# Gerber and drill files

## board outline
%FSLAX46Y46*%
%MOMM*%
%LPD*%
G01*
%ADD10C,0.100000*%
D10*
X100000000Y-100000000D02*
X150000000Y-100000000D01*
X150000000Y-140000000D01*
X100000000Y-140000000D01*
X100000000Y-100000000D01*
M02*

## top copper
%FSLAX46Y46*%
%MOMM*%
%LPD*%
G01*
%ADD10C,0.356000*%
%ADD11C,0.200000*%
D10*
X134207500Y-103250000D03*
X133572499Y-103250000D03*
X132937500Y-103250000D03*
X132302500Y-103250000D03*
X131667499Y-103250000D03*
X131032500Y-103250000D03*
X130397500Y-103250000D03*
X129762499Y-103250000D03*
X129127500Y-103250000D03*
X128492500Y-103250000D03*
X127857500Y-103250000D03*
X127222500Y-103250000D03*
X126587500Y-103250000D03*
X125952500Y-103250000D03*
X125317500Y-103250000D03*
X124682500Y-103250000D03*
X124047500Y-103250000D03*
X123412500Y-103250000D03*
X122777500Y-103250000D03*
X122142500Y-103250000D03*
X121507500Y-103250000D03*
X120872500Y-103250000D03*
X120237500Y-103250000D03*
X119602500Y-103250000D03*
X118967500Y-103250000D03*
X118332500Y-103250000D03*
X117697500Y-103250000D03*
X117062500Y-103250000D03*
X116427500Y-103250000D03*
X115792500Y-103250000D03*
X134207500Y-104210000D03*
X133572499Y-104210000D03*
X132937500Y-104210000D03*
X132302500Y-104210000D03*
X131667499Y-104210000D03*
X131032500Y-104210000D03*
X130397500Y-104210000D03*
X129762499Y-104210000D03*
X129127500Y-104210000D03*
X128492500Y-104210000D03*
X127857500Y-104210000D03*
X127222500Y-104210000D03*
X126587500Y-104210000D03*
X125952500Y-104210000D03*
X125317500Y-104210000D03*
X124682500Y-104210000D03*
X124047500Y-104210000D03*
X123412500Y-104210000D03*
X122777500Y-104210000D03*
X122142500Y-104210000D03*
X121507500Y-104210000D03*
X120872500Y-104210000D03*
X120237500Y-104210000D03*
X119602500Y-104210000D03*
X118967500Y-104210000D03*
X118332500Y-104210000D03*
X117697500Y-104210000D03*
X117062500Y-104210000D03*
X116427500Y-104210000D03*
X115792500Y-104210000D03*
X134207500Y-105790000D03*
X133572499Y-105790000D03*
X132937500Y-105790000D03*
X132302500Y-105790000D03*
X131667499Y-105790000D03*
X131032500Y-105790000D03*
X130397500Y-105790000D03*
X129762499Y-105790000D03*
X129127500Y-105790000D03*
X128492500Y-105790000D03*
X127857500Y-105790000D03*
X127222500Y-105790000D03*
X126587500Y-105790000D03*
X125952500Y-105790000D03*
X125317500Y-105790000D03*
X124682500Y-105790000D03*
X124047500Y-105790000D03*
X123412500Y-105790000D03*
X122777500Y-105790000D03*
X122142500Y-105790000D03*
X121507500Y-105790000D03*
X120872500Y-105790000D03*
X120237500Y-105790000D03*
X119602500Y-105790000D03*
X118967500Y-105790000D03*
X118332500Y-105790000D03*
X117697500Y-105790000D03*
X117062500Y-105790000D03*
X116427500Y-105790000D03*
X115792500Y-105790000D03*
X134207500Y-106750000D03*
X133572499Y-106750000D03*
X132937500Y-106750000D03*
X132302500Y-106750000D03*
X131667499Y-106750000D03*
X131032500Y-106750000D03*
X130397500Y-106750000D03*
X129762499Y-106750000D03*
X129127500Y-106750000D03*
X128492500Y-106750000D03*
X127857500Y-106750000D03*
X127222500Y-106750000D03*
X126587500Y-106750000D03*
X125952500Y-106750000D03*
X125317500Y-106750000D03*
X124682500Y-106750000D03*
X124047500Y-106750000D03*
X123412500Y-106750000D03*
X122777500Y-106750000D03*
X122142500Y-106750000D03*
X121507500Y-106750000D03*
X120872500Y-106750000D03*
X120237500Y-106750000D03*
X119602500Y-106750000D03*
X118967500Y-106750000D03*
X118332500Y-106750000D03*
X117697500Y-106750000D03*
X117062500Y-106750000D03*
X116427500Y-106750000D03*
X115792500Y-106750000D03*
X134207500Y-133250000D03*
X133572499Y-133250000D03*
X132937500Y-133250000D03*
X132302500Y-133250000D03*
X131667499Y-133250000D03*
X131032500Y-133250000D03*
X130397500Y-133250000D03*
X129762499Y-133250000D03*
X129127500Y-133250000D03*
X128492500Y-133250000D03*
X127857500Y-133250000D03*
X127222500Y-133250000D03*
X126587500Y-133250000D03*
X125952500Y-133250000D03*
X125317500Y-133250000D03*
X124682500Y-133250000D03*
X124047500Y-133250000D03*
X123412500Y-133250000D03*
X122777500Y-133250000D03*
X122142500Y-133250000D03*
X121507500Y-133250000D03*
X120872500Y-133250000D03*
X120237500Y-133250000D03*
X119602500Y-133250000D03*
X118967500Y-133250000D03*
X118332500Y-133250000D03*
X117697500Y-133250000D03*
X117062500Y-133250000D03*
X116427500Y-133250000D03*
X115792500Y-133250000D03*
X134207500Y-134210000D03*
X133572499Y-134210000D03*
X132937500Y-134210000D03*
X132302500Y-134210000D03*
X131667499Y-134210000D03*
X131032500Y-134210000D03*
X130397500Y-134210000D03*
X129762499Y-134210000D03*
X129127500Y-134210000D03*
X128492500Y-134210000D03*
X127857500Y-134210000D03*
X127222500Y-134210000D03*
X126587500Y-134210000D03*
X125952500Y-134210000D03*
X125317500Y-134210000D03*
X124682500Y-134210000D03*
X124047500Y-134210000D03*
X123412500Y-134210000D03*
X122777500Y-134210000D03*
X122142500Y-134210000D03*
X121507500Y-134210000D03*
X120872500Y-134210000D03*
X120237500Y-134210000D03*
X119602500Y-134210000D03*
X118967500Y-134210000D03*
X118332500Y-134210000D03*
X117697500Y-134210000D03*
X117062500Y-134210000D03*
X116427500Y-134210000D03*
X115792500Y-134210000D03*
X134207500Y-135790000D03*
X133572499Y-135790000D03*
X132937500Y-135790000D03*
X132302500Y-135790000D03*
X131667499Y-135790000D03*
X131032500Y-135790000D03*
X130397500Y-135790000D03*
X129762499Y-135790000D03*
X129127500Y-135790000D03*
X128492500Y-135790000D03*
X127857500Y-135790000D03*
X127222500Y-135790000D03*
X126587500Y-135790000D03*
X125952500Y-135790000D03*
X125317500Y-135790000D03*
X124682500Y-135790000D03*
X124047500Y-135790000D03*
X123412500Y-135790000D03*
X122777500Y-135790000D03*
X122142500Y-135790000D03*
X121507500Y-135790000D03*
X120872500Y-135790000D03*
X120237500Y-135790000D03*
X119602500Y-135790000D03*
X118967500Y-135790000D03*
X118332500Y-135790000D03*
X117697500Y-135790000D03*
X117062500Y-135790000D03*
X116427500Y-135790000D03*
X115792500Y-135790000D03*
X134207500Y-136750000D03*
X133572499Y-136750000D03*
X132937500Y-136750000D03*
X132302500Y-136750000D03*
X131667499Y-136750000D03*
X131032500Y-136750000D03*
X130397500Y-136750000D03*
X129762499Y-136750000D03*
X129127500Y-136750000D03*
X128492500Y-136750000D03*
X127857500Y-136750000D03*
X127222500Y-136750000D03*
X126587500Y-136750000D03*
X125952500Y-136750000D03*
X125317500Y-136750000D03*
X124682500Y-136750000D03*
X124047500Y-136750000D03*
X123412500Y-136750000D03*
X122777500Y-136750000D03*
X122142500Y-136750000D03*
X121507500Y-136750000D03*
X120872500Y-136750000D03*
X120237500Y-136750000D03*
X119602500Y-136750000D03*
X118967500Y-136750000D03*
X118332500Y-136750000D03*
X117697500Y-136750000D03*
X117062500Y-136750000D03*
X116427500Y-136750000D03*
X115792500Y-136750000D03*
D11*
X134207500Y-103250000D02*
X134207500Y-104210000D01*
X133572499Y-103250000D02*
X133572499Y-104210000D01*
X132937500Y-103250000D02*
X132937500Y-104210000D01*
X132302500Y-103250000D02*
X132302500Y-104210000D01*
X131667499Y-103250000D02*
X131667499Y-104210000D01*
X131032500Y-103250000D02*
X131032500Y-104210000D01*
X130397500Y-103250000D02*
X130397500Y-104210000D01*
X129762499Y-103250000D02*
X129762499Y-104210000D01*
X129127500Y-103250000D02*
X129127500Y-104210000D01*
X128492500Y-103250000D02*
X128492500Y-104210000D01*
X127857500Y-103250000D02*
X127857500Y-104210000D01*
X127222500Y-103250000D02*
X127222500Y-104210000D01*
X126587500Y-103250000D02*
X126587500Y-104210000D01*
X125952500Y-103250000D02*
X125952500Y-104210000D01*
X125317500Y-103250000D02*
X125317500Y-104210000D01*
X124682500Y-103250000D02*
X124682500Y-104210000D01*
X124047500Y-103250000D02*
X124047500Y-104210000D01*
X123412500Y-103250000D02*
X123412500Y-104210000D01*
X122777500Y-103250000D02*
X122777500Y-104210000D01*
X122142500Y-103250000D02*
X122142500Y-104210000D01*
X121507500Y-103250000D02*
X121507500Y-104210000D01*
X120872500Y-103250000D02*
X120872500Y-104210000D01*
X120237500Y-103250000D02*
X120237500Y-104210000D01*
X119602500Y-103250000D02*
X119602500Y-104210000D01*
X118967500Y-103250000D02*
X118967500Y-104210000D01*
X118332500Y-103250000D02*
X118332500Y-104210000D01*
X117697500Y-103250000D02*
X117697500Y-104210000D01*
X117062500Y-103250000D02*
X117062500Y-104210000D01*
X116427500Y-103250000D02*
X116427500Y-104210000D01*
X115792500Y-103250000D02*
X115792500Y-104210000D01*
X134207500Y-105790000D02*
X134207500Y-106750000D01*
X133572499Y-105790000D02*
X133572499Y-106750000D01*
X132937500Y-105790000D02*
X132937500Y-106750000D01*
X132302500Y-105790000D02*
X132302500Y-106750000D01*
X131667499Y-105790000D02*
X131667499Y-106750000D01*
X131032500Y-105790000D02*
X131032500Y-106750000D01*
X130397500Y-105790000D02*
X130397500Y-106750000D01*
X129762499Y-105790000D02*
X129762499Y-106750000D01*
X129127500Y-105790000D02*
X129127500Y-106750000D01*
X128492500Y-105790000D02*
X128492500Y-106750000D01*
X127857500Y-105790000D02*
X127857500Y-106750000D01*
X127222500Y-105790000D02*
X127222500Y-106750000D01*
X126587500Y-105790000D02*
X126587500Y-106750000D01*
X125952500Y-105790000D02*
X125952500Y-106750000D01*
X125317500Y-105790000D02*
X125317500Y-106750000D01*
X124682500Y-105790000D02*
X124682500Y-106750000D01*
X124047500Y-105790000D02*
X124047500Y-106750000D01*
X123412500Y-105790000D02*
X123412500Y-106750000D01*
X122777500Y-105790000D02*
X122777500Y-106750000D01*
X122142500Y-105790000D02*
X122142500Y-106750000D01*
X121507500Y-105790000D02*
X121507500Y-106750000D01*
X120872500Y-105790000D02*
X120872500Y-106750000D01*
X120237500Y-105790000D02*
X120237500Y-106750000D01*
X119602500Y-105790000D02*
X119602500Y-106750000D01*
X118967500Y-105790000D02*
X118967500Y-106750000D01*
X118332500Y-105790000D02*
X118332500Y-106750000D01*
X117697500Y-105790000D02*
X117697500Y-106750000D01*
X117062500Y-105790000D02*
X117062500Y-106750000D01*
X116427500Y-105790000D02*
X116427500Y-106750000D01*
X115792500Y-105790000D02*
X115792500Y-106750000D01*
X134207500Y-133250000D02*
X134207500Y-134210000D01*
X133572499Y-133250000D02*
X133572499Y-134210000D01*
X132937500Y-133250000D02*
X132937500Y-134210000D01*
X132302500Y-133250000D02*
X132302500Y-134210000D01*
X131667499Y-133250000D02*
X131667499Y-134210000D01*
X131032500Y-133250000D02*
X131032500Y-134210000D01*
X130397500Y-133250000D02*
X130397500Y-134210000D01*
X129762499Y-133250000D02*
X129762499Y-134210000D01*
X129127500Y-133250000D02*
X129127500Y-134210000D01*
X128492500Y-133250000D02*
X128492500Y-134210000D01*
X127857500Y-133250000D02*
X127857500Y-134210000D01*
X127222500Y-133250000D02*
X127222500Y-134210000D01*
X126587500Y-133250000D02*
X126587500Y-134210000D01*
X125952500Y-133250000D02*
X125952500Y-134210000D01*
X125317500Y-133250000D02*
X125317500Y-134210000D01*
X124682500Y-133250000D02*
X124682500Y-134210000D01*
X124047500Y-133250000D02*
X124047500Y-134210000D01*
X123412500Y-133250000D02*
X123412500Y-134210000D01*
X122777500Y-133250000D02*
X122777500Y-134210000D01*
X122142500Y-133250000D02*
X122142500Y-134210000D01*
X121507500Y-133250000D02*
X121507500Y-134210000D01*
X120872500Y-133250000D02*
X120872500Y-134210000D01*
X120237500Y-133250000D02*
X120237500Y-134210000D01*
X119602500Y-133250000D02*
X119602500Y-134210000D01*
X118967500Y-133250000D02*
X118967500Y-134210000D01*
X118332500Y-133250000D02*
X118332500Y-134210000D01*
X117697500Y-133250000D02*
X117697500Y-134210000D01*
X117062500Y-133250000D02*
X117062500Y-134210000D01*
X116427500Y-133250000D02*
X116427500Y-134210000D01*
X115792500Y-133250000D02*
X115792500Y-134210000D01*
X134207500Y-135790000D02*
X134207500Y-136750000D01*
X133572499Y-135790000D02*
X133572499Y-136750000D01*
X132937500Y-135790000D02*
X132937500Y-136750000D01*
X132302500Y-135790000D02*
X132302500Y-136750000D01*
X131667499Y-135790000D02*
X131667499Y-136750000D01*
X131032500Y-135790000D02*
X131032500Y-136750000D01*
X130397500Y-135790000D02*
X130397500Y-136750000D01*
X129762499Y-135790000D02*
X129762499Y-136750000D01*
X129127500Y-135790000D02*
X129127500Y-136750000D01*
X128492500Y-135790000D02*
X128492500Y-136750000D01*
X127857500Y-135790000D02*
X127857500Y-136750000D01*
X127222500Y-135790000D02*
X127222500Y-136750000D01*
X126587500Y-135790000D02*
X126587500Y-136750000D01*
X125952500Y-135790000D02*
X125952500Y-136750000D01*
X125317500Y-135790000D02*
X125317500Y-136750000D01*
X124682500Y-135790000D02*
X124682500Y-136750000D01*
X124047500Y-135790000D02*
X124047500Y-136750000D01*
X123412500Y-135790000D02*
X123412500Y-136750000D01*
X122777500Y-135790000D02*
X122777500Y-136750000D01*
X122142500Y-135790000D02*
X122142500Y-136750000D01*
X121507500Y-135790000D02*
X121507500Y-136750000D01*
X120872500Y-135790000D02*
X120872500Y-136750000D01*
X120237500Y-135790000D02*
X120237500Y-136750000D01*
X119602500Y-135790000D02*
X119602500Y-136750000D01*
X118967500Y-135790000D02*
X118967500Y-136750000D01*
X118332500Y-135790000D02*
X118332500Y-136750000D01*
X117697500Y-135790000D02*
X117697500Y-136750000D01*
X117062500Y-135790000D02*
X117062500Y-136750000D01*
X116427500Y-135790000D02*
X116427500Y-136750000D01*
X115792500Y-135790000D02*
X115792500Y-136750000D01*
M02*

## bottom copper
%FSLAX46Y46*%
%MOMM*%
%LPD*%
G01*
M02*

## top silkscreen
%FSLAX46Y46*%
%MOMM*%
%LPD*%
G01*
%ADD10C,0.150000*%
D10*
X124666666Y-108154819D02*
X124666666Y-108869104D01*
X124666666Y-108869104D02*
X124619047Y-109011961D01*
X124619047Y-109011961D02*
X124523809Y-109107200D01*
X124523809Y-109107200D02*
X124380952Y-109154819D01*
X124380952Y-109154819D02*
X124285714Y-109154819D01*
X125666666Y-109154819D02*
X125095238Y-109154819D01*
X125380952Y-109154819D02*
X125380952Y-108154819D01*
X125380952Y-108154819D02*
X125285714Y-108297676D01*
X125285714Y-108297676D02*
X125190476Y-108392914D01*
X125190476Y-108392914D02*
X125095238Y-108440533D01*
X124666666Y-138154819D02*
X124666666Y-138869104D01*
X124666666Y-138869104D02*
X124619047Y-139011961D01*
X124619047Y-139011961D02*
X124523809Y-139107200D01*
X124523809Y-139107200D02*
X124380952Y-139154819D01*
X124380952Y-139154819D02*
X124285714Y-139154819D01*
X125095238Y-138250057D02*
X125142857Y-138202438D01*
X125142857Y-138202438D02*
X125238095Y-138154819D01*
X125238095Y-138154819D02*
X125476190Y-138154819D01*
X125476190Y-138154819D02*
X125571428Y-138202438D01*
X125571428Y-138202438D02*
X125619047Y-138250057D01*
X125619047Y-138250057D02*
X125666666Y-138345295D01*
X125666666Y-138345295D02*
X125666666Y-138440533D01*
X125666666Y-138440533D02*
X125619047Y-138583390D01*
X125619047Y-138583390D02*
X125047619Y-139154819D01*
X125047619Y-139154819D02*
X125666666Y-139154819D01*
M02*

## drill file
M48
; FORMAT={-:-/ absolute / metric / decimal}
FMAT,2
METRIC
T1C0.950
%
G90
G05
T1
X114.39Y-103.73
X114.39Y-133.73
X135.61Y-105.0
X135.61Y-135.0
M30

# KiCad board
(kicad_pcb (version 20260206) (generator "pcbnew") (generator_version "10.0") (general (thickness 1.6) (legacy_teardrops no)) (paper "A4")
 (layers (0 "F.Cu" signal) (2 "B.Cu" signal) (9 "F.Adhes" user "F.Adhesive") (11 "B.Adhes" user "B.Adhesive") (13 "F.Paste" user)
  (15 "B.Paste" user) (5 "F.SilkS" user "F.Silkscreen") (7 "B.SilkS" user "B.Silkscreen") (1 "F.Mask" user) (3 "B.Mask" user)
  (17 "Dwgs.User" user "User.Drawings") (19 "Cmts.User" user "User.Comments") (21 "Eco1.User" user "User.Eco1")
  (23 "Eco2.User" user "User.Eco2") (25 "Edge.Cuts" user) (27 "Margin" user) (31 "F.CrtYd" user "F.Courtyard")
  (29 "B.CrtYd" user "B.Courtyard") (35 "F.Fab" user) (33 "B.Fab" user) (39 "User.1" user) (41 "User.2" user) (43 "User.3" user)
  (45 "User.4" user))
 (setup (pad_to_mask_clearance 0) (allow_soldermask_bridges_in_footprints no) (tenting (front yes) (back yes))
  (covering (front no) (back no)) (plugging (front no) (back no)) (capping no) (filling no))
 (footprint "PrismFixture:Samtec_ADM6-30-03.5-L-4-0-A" (layer "F.Cu") (at 125 105)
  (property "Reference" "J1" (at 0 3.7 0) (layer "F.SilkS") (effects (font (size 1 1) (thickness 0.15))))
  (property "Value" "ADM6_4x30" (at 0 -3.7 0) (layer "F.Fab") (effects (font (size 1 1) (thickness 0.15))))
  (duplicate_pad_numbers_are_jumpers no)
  (pad "" np_thru_hole circle (at -10.61 -1.27) (size 0.95 0.95) (drill 0.95) (layers "*.Cu" "*.Mask"))
  (pad "" np_thru_hole circle (at 10.61 0) (size 0.95 0.95) (drill 0.95) (layers "*.Cu" "*.Mask"))
  (pad "A01" smd circle (at 9.2075 -1.75) (size 0.356 0.356) (layers "F.Cu" "F.Mask" "F.Paste") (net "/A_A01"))
  (pad "A02" smd circle (at 8.572499 -1.75) (size 0.356 0.356) (layers "F.Cu" "F.Mask" "F.Paste") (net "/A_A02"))
  (pad "A03" smd circle (at 7.9375 -1.75) (size 0.356 0.356) (layers "F.Cu" "F.Mask" "F.Paste") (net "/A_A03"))
  (pad "A04" smd circle (at 7.3025 -1.75) (size 0.356 0.356) (layers "F.Cu" "F.Mask" "F.Paste") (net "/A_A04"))
  (pad "A05" smd circle (at 6.667499 -1.75) (size 0.356 0.356) (layers "F.Cu" "F.Mask" "F.Paste") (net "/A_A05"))
  (pad "A06" smd circle (at 6.0325 -1.75) (size 0.356 0.356) (layers "F.Cu" "F.Mask" "F.Paste") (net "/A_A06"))
  (pad "A07" smd circle (at 5.3975 -1.75) (size 0.356 0.356) (layers "F.Cu" "F.Mask" "F.Paste") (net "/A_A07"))
  (pad "A08" smd circle (at 4.762499 -1.75) (size 0.356 0.356) (layers "F.Cu" "F.Mask" "F.Paste") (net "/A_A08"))
  (pad "A09" smd circle (at 4.1275 -1.75) (size 0.356 0.356) (layers "F.Cu" "F.Mask" "F.Paste") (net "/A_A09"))
  (pad "A10" smd circle (at 3.4925 -1.75) (size 0.356 0.356) (layers "F.Cu" "F.Mask" "F.Paste") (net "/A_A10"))
  (pad "A11" smd circle (at 2.8575 -1.75) (size 0.356 0.356) (layers "F.Cu" "F.Mask" "F.Paste") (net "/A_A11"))
  (pad "A12" smd circle (at 2.2225 -1.75) (size 0.356 0.356) (layers "F.Cu" "F.Mask" "F.Paste") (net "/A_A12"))
  (pad "A13" smd circle (at 1.5875 -1.75) (size 0.356 0.356) (layers "F.Cu" "F.Mask" "F.Paste") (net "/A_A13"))
  (pad "A14" smd circle (at 0.9525 -1.75) (size 0.356 0.356) (layers "F.Cu" "F.Mask" "F.Paste") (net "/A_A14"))
  (pad "A15" smd circle (at 0.3175 -1.75) (size 0.356 0.356) (layers "F.Cu" "F.Mask" "F.Paste") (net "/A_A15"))
  (pad "A16" smd circle (at -0.3175 -1.75) (size 0.356 0.356) (layers "F.Cu" "F.Mask" "F.Paste") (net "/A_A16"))
  (pad "A17" smd circle (at -0.9525 -1.75) (size 0.356 0.356) (layers "F.Cu" "F.Mask" "F.Paste") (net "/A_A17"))
  (pad "A18" smd circle (at -1.5875 -1.75) (size 0.356 0.356) (layers "F.Cu" "F.Mask" "F.Paste") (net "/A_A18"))
  (pad "A19" smd circle (at -2.2225 -1.75) (size 0.356 0.356) (layers "F.Cu" "F.Mask" "F.Paste") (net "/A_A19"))
  (pad "A20" smd circle (at -2.8575 -1.75) (size 0.356 0.356) (layers "F.Cu" "F.Mask" "F.Paste") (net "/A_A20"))
  (pad "A21" smd circle (at -3.4925 -1.75) (size 0.356 0.356) (layers "F.Cu" "F.Mask" "F.Paste") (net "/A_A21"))
  (pad "A22" smd circle (at -4.1275 -1.75) (size 0.356 0.356) (layers "F.Cu" "F.Mask" "F.Paste") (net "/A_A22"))
  (pad "A23" smd circle (at -4.7625 -1.75) (size 0.356 0.356) (layers "F.Cu" "F.Mask" "F.Paste") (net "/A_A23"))
  (pad "A24" smd circle (at -5.3975 -1.75) (size 0.356 0.356) (layers "F.Cu" "F.Mask" "F.Paste") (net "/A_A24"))
  (pad "A25" smd circle (at -6.0325 -1.75) (size 0.356 0.356) (layers "F.Cu" "F.Mask" "F.Paste") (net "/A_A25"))
  (pad "A26" smd circle (at -6.6675 -1.75) (size 0.356 0.356) (layers "F.Cu" "F.Mask" "F.Paste") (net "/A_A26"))
  (pad "A27" smd circle (at -7.3025 -1.75) (size 0.356 0.356) (layers "F.Cu" "F.Mask" "F.Paste") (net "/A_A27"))
  (pad "A28" smd circle (at -7.9375 -1.75) (size 0.356 0.356) (layers "F.Cu" "F.Mask" "F.Paste") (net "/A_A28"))
  (pad "A29" smd circle (at -8.5725 -1.75) (size 0.356 0.356) (layers "F.Cu" "F.Mask" "F.Paste") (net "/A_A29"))
  (pad "A30" smd circle (at -9.2075 -1.75) (size 0.356 0.356) (layers "F.Cu" "F.Mask" "F.Paste") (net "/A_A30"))
  (pad "B01" smd circle (at 9.2075 -0.79) (size 0.356 0.356) (layers "F.Cu" "F.Mask" "F.Paste") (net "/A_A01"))
  (pad "B02" smd circle (at 8.572499 -0.79) (size 0.356 0.356) (layers "F.Cu" "F.Mask" "F.Paste") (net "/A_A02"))
  (pad "B03" smd circle (at 7.9375 -0.79) (size 0.356 0.356) (layers "F.Cu" "F.Mask" "F.Paste") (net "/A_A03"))
  (pad "B04" smd circle (at 7.3025 -0.79) (size 0.356 0.356) (layers "F.Cu" "F.Mask" "F.Paste") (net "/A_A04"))
  (pad "B05" smd circle (at 6.667499 -0.79) (size 0.356 0.356) (layers "F.Cu" "F.Mask" "F.Paste") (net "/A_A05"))
  (pad "B06" smd circle (at 6.0325 -0.79) (size 0.356 0.356) (layers "F.Cu" "F.Mask" "F.Paste") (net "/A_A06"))
  (pad "B07" smd circle (at 5.3975 -0.79) (size 0.356 0.356) (layers "F.Cu" "F.Mask" "F.Paste") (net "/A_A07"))
  (pad "B08" smd circle (at 4.762499 -0.79) (size 0.356 0.356) (layers "F.Cu" "F.Mask" "F.Paste") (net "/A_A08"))
  (pad "B09" smd circle (at 4.1275 -0.79) (size 0.356 0.356) (layers "F.Cu" "F.Mask" "F.Paste") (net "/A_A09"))
  (pad "B10" smd circle (at 3.4925 -0.79) (size 0.356 0.356) (layers "F.Cu" "F.Mask" "F.Paste") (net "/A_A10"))
  (pad "B11" smd circle (at 2.8575 -0.79) (size 0.356 0.356) (layers "F.Cu" "F.Mask" "F.Paste") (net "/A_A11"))
  (pad "B12" smd circle (at 2.2225 -0.79) (size 0.356 0.356) (layers "F.Cu" "F.Mask" "F.Paste") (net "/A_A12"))
  (pad "B13" smd circle (at 1.5875 -0.79) (size 0.356 0.356) (layers "F.Cu" "F.Mask" "F.Paste") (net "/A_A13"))
  (pad "B14" smd circle (at 0.9525 -0.79) (size 0.356 0.356) (layers "F.Cu" "F.Mask" "F.Paste") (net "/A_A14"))
  (pad "B15" smd circle (at 0.3175 -0.79) (size 0.356 0.356) (layers "F.Cu" "F.Mask" "F.Paste") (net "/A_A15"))
  (pad "B16" smd circle (at -0.3175 -0.79) (size 0.356 0.356) (layers "F.Cu" "F.Mask" "F.Paste") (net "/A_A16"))
  (pad "B17" smd circle (at -0.9525 -0.79) (size 0.356 0.356) (layers "F.Cu" "F.Mask" "F.Paste") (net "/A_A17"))
  (pad "B18" smd circle (at -1.5875 -0.79) (size 0.356 0.356) (layers "F.Cu" "F.Mask" "F.Paste") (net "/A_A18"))
  (pad "B19" smd circle (at -2.2225 -0.79) (size 0.356 0.356) (layers "F.Cu" "F.Mask" "F.Paste") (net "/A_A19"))
  (pad "B20" smd circle (at -2.8575 -0.79) (size 0.356 0.356) (layers "F.Cu" "F.Mask" "F.Paste") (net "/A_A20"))
  (pad "B21" smd circle (at -3.4925 -0.79) (size 0.356 0.356) (layers "F.Cu" "F.Mask" "F.Paste") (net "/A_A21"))
  (pad "B22" smd circle (at -4.1275 -0.79) (size 0.356 0.356) (layers "F.Cu" "F.Mask" "F.Paste") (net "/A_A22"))
  (pad "B23" smd circle (at -4.7625 -0.79) (size 0.356 0.356) (layers "F.Cu" "F.Mask" "F.Paste") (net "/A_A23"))
  (pad "B24" smd circle (at -5.3975 -0.79) (size 0.356 0.356) (layers "F.Cu" "F.Mask" "F.Paste") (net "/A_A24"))
  (pad "B25" smd circle (at -6.0325 -0.79) (size 0.356 0.356) (layers "F.Cu" "F.Mask" "F.Paste") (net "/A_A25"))
  (pad "B26" smd circle (at -6.6675 -0.79) (size 0.356 0.356) (layers "F.Cu" "F.Mask" "F.Paste") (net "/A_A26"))
  (pad "B27" smd circle (at -7.3025 -0.79) (size 0.356 0.356) (layers "F.Cu" "F.Mask" "F.Paste") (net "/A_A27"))
  (pad "B28" smd circle (at -7.9375 -0.79) (size 0.356 0.356) (layers "F.Cu" "F.Mask" "F.Paste") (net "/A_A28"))
  (pad "B29" smd circle (at -8.5725 -0.79) (size 0.356 0.356) (layers "F.Cu" "F.Mask" "F.Paste") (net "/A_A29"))
  (pad "B30" smd circle (at -9.2075 -0.79) (size 0.356 0.356) (layers "F.Cu" "F.Mask" "F.Paste") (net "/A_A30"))
  (pad "C01" smd circle (at 9.2075 0.79) (size 0.356 0.356) (layers "F.Cu" "F.Mask" "F.Paste") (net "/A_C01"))
  (pad "C02" smd circle (at 8.572499 0.79) (size 0.356 0.356) (layers "F.Cu" "F.Mask" "F.Paste") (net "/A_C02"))
  (pad "C03" smd circle (at 7.9375 0.79) (size 0.356 0.356) (layers "F.Cu" "F.Mask" "F.Paste") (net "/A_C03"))
  (pad "C04" smd circle (at 7.3025 0.79) (size 0.356 0.356) (layers "F.Cu" "F.Mask" "F.Paste") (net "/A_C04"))
  (pad "C05" smd circle (at 6.667499 0.79) (size 0.356 0.356) (layers "F.Cu" "F.Mask" "F.Paste") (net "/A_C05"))
  (pad "C06" smd circle (at 6.0325 0.79) (size 0.356 0.356) (layers "F.Cu" "F.Mask" "F.Paste") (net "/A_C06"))
  (pad "C07" smd circle (at 5.3975 0.79) (size 0.356 0.356) (layers "F.Cu" "F.Mask" "F.Paste") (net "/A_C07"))
  (pad "C08" smd circle (at 4.762499 0.79) (size 0.356 0.356) (layers "F.Cu" "F.Mask" "F.Paste") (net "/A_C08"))
  (pad "C09" smd circle (at 4.1275 0.79) (size 0.356 0.356) (layers "F.Cu" "F.Mask" "F.Paste") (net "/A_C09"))
  (pad "C10" smd circle (at 3.4925 0.79) (size 0.356 0.356) (layers "F.Cu" "F.Mask" "F.Paste") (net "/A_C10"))
  (pad "C11" smd circle (at 2.8575 0.79) (size 0.356 0.356) (layers "F.Cu" "F.Mask" "F.Paste") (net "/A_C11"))
  (pad "C12" smd circle (at 2.2225 0.79) (size 0.356 0.356) (layers "F.Cu" "F.Mask" "F.Paste") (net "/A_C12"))
  (pad "C13" smd circle (at 1.5875 0.79) (size 0.356 0.356) (layers "F.Cu" "F.Mask" "F.Paste") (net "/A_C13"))
  (pad "C14" smd circle (at 0.9525 0.79) (size 0.356 0.356) (layers "F.Cu" "F.Mask" "F.Paste") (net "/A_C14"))
  (pad "C15" smd circle (at 0.3175 0.79) (size 0.356 0.356) (layers "F.Cu" "F.Mask" "F.Paste") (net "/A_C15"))
  (pad "C16" smd circle (at -0.3175 0.79) (size 0.356 0.356) (layers "F.Cu" "F.Mask" "F.Paste") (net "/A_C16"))
  (pad "C17" smd circle (at -0.9525 0.79) (size 0.356 0.356) (layers "F.Cu" "F.Mask" "F.Paste") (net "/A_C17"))
  (pad "C18" smd circle (at -1.5875 0.79) (size 0.356 0.356) (layers "F.Cu" "F.Mask" "F.Paste") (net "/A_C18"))
  (pad "C19" smd circle (at -2.2225 0.79) (size 0.356 0.356) (layers "F.Cu" "F.Mask" "F.Paste") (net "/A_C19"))
  (pad "C20" smd circle (at -2.8575 0.79) (size 0.356 0.356) (layers "F.Cu" "F.Mask" "F.Paste") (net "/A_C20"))
  (pad "C21" smd circle (at -3.4925 0.79) (size 0.356 0.356) (layers "F.Cu" "F.Mask" "F.Paste") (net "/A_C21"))
  (pad "C22" smd circle (at -4.1275 0.79) (size 0.356 0.356) (layers "F.Cu" "F.Mask" "F.Paste") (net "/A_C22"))
  (pad "C23" smd circle (at -4.7625 0.79) (size 0.356 0.356) (layers "F.Cu" "F.Mask" "F.Paste") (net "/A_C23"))
  (pad "C24" smd circle (at -5.3975 0.79) (size 0.356 0.356) (layers "F.Cu" "F.Mask" "F.Paste") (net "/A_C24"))
  (pad "C25" smd circle (at -6.0325 0.79) (size 0.356 0.356) (layers "F.Cu" "F.Mask" "F.Paste") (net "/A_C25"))
  (pad "C26" smd circle (at -6.6675 0.79) (size 0.356 0.356) (layers "F.Cu" "F.Mask" "F.Paste") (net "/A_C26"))
  (pad "C27" smd circle (at -7.3025 0.79) (size 0.356 0.356) (layers "F.Cu" "F.Mask" "F.Paste") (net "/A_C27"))
  (pad "C28" smd circle (at -7.9375 0.79) (size 0.356 0.356) (layers "F.Cu" "F.Mask" "F.Paste") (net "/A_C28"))
  (pad "C29" smd circle (at -8.5725 0.79) (size 0.356 0.356) (layers "F.Cu" "F.Mask" "F.Paste") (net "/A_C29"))
  (pad "C30" smd circle (at -9.2075 0.79) (size 0.356 0.356) (layers "F.Cu" "F.Mask" "F.Paste") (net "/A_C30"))
  (pad "D01" smd circle (at 9.2075 1.75) (size 0.356 0.356) (layers "F.Cu" "F.Mask" "F.Paste") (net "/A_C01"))
  (pad "D02" smd circle (at 8.572499 1.75) (size 0.356 0.356) (layers "F.Cu" "F.Mask" "F.Paste") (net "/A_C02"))
  (pad "D03" smd circle (at 7.9375 1.75) (size 0.356 0.356) (layers "F.Cu" "F.Mask" "F.Paste") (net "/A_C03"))
  (pad "D04" smd circle (at 7.3025 1.75) (size 0.356 0.356) (layers "F.Cu" "F.Mask" "F.Paste") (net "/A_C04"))
  (pad "D05" smd circle (at 6.667499 1.75) (size 0.356 0.356) (layers "F.Cu" "F.Mask" "F.Paste") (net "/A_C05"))
  (pad "D06" smd circle (at 6.0325 1.75) (size 0.356 0.356) (layers "F.Cu" "F.Mask" "F.Paste") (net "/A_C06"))
  (pad "D07" smd circle (at 5.3975 1.75) (size 0.356 0.356) (layers "F.Cu" "F.Mask" "F.Paste") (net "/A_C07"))
  (pad "D08" smd circle (at 4.762499 1.75) (size 0.356 0.356) (layers "F.Cu" "F.Mask" "F.Paste") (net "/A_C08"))
  (pad "D09" smd circle (at 4.1275 1.75) (size 0.356 0.356) (layers "F.Cu" "F.Mask" "F.Paste") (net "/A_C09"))
  (pad "D10" smd circle (at 3.4925 1.75) (size 0.356 0.356) (layers "F.Cu" "F.Mask" "F.Paste") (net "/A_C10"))
  (pad "D11" smd circle (at 2.8575 1.75) (size 0.356 0.356) (layers "F.Cu" "F.Mask" "F.Paste") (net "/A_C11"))
  (pad "D12" smd circle (at 2.2225 1.75) (size 0.356 0.356) (layers "F.Cu" "F.Mask" "F.Paste") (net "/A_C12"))
  (pad "D13" smd circle (at 1.5875 1.75) (size 0.356 0.356) (layers "F.Cu" "F.Mask" "F.Paste") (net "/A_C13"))
  (pad "D14" smd circle (at 0.9525 1.75) (size 0.356 0.356) (layers "F.Cu" "F.Mask" "F.Paste") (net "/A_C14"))
  (pad "D15" smd circle (at 0.3175 1.75) (size 0.356 0.356) (layers "F.Cu" "F.Mask" "F.Paste") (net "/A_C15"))
  (pad "D16" smd circle (at -0.3175 1.75) (size 0.356 0.356) (layers "F.Cu" "F.Mask" "F.Paste") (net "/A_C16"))
  (pad "D17" smd circle (at -0.9525 1.75) (size 0.356 0.356) (layers "F.Cu" "F.Mask" "F.Paste") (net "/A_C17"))
  (pad "D18" smd circle (at -1.5875 1.75) (size 0.356 0.356) (layers "F.Cu" "F.Mask" "F.Paste") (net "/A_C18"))
  (pad "D19" smd circle (at -2.2225 1.75) (size 0.356 0.356) (layers "F.Cu" "F.Mask" "F.Paste") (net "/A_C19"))
  (pad "D20" smd circle (at -2.8575 1.75) (size 0.356 0.356) (layers "F.Cu" "F.Mask" "F.Paste") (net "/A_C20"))
  (pad "D21" smd circle (at -3.4925 1.75) (size 0.356 0.356) (layers "F.Cu" "F.Mask" "F.Paste") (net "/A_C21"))
  (pad "D22" smd circle (at -4.1275 1.75) (size 0.356 0.356) (layers "F.Cu" "F.Mask" "F.Paste") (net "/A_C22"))
  (pad "D23" smd circle (at -4.7625 1.75) (size 0.356 0.356) (layers "F.Cu" "F.Mask" "F.Paste") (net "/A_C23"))
  (pad "D24" smd circle (at -5.3975 1.75) (size 0.356 0.356) (layers "F.Cu" "F.Mask" "F.Paste") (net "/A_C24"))
  (pad "D25" smd circle (at -6.0325 1.75) (size 0.356 0.356) (layers "F.Cu" "F.Mask" "F.Paste") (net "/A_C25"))
  (pad "D26" smd circle (at -6.6675 1.75) (size 0.356 0.356) (layers "F.Cu" "F.Mask" "F.Paste") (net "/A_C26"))
  (pad "D27" smd circle (at -7.3025 1.75) (size 0.356 0.356) (layers "F.Cu" "F.Mask" "F.Paste") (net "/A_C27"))
  (pad "D28" smd circle (at -7.9375 1.75) (size 0.356 0.356) (layers "F.Cu" "F.Mask" "F.Paste") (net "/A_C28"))
  (pad "D29" smd circle (at -8.5725 1.75) (size 0.356 0.356) (layers "F.Cu" "F.Mask" "F.Paste") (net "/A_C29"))
  (pad "D30" smd circle (at -9.2075 1.75) (size 0.356 0.356) (layers "F.Cu" "F.Mask" "F.Paste") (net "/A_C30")))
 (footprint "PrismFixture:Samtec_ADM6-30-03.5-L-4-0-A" (layer "F.Cu") (at 125 135)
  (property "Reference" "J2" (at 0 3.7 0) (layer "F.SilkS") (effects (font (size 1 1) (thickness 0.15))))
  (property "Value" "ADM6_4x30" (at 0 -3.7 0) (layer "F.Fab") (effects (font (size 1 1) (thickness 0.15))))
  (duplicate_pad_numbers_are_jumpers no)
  (pad "" np_thru_hole circle (at -10.61 -1.270001) (size 0.95 0.95) (drill 0.95) (layers "*.Cu" "*.Mask"))
  (pad "" np_thru_hole circle (at 10.61 0) (size 0.95 0.95) (drill 0.95) (layers "*.Cu" "*.Mask"))
  (pad "A01" smd circle (at 9.2075 -1.75) (size 0.356 0.356) (layers "F.Cu" "F.Mask" "F.Paste") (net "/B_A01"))
  (pad "A02" smd circle (at 8.572499 -1.75) (size 0.356 0.356) (layers "F.Cu" "F.Mask" "F.Paste") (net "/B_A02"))
  (pad "A03" smd circle (at 7.9375 -1.75) (size 0.356 0.356) (layers "F.Cu" "F.Mask" "F.Paste") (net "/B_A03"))
  (pad "A04" smd circle (at 7.3025 -1.75) (size 0.356 0.356) (layers "F.Cu" "F.Mask" "F.Paste") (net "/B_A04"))
  (pad "A05" smd circle (at 6.667499 -1.75) (size 0.356 0.356) (layers "F.Cu" "F.Mask" "F.Paste") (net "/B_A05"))
  (pad "A06" smd circle (at 6.0325 -1.75) (size 0.356 0.356) (layers "F.Cu" "F.Mask" "F.Paste") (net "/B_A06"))
  (pad "A07" smd circle (at 5.3975 -1.75) (size 0.356 0.356) (layers "F.Cu" "F.Mask" "F.Paste") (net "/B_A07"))
  (pad "A08" smd circle (at 4.762499 -1.75) (size 0.356 0.356) (layers "F.Cu" "F.Mask" "F.Paste") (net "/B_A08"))
  (pad "A09" smd circle (at 4.1275 -1.75) (size 0.356 0.356) (layers "F.Cu" "F.Mask" "F.Paste") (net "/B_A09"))
  (pad "A10" smd circle (at 3.4925 -1.75) (size 0.356 0.356) (layers "F.Cu" "F.Mask" "F.Paste") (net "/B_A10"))
  (pad "A11" smd circle (at 2.8575 -1.75) (size 0.356 0.356) (layers "F.Cu" "F.Mask" "F.Paste") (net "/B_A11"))
  (pad "A12" smd circle (at 2.2225 -1.75) (size 0.356 0.356) (layers "F.Cu" "F.Mask" "F.Paste") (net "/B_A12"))
  (pad "A13" smd circle (at 1.5875 -1.75) (size 0.356 0.356) (layers "F.Cu" "F.Mask" "F.Paste") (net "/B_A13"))
  (pad "A14" smd circle (at 0.9525 -1.75) (size 0.356 0.356) (layers "F.Cu" "F.Mask" "F.Paste") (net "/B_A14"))
  (pad "A15" smd circle (at 0.3175 -1.75) (size 0.356 0.356) (layers "F.Cu" "F.Mask" "F.Paste") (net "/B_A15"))
  (pad "A16" smd circle (at -0.3175 -1.75) (size 0.356 0.356) (layers "F.Cu" "F.Mask" "F.Paste") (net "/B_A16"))
  (pad "A17" smd circle (at -0.9525 -1.75) (size 0.356 0.356) (layers "F.Cu" "F.Mask" "F.Paste") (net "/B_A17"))
  (pad "A18" smd circle (at -1.5875 -1.75) (size 0.356 0.356) (layers "F.Cu" "F.Mask" "F.Paste") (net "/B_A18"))
  (pad "A19" smd circle (at -2.2225 -1.75) (size 0.356 0.356) (layers "F.Cu" "F.Mask" "F.Paste") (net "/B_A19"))
  (pad "A20" smd circle (at -2.8575 -1.75) (size 0.356 0.356) (layers "F.Cu" "F.Mask" "F.Paste") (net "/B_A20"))
  (pad "A21" smd circle (at -3.4925 -1.75) (size 0.356 0.356) (layers "F.Cu" "F.Mask" "F.Paste") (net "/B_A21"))
  (pad "A22" smd circle (at -4.1275 -1.75) (size 0.356 0.356) (layers "F.Cu" "F.Mask" "F.Paste") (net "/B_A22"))
  (pad "A23" smd circle (at -4.7625 -1.75) (size 0.356 0.356) (layers "F.Cu" "F.Mask" "F.Paste") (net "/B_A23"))
  (pad "A24" smd circle (at -5.3975 -1.75) (size 0.356 0.356) (layers "F.Cu" "F.Mask" "F.Paste") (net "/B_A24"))
  (pad "A25" smd circle (at -6.0325 -1.75) (size 0.356 0.356) (layers "F.Cu" "F.Mask" "F.Paste") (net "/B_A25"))
  (pad "A26" smd circle (at -6.6675 -1.75) (size 0.356 0.356) (layers "F.Cu" "F.Mask" "F.Paste") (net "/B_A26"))
  (pad "A27" smd circle (at -7.3025 -1.75) (size 0.356 0.356) (layers "F.Cu" "F.Mask" "F.Paste") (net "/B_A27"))
  (pad "A28" smd circle (at -7.9375 -1.75) (size 0.356 0.356) (layers "F.Cu" "F.Mask" "F.Paste") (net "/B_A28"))
  (pad "A29" smd circle (at -8.5725 -1.75) (size 0.356 0.356) (layers "F.Cu" "F.Mask" "F.Paste") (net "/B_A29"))
  (pad "A30" smd circle (at -9.2075 -1.75) (size 0.356 0.356) (layers "F.Cu" "F.Mask" "F.Paste") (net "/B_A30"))
  (pad "B01" smd circle (at 9.2075 -0.79) (size 0.356 0.356) (layers "F.Cu" "F.Mask" "F.Paste") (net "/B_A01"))
  (pad "B02" smd circle (at 8.572499 -0.79) (size 0.356 0.356) (layers "F.Cu" "F.Mask" "F.Paste") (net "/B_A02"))
  (pad "B03" smd circle (at 7.9375 -0.79) (size 0.356 0.356) (layers "F.Cu" "F.Mask" "F.Paste") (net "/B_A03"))
  (pad "B04" smd circle (at 7.3025 -0.79) (size 0.356 0.356) (layers "F.Cu" "F.Mask" "F.Paste") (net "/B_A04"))
  (pad "B05" smd circle (at 6.667499 -0.79) (size 0.356 0.356) (layers "F.Cu" "F.Mask" "F.Paste") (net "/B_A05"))
  (pad "B06" smd circle (at 6.0325 -0.79) (size 0.356 0.356) (layers "F.Cu" "F.Mask" "F.Paste") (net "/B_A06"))
  (pad "B07" smd circle (at 5.3975 -0.79) (size 0.356 0.356) (layers "F.Cu" "F.Mask" "F.Paste") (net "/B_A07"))
  (pad "B08" smd circle (at 4.762499 -0.79) (size 0.356 0.356) (layers "F.Cu" "F.Mask" "F.Paste") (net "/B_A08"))
  (pad "B09" smd circle (at 4.1275 -0.79) (size 0.356 0.356) (layers "F.Cu" "F.Mask" "F.Paste") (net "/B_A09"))
  (pad "B10" smd circle (at 3.4925 -0.79) (size 0.356 0.356) (layers "F.Cu" "F.Mask" "F.Paste") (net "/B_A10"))
  (pad "B11" smd circle (at 2.8575 -0.79) (size 0.356 0.356) (layers "F.Cu" "F.Mask" "F.Paste") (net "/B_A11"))
  (pad "B12" smd circle (at 2.2225 -0.79) (size 0.356 0.356) (layers "F.Cu" "F.Mask" "F.Paste") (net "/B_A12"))
  (pad "B13" smd circle (at 1.5875 -0.79) (size 0.356 0.356) (layers "F.Cu" "F.Mask" "F.Paste") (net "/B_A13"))
  (pad "B14" smd circle (at 0.9525 -0.79) (size 0.356 0.356) (layers "F.Cu" "F.Mask" "F.Paste") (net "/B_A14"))
  (pad "B15" smd circle (at 0.3175 -0.79) (size 0.356 0.356) (layers "F.Cu" "F.Mask" "F.Paste") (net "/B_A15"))
  (pad "B16" smd circle (at -0.3175 -0.79) (size 0.356 0.356) (layers "F.Cu" "F.Mask" "F.Paste") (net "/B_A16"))
  (pad "B17" smd circle (at -0.9525 -0.79) (size 0.356 0.356) (layers "F.Cu" "F.Mask" "F.Paste") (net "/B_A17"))
  (pad "B18" smd circle (at -1.5875 -0.79) (size 0.356 0.356) (layers "F.Cu" "F.Mask" "F.Paste") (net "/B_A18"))
  (pad "B19" smd circle (at -2.2225 -0.79) (size 0.356 0.356) (layers "F.Cu" "F.Mask" "F.Paste") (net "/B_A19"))
  (pad "B20" smd circle (at -2.8575 -0.79) (size 0.356 0.356) (layers "F.Cu" "F.Mask" "F.Paste") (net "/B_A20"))
  (pad "B21" smd circle (at -3.4925 -0.79) (size 0.356 0.356) (layers "F.Cu" "F.Mask" "F.Paste") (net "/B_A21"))
  (pad "B22" smd circle (at -4.1275 -0.79) (size 0.356 0.356) (layers "F.Cu" "F.Mask" "F.Paste") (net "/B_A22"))
  (pad "B23" smd circle (at -4.7625 -0.79) (size 0.356 0.356) (layers "F.Cu" "F.Mask" "F.Paste") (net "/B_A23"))
  (pad "B24" smd circle (at -5.3975 -0.79) (size 0.356 0.356) (layers "F.Cu" "F.Mask" "F.Paste") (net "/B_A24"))
  (pad "B25" smd circle (at -6.0325 -0.79) (size 0.356 0.356) (layers "F.Cu" "F.Mask" "F.Paste") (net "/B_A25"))
  (pad "B26" smd circle (at -6.6675 -0.79) (size 0.356 0.356) (layers "F.Cu" "F.Mask" "F.Paste") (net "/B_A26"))
  (pad "B27" smd circle (at -7.3025 -0.79) (size 0.356 0.356) (layers "F.Cu" "F.Mask" "F.Paste") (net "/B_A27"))
  (pad "B28" smd circle (at -7.9375 -0.79) (size 0.356 0.356) (layers "F.Cu" "F.Mask" "F.Paste") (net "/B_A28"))
  (pad "B29" smd circle (at -8.5725 -0.79) (size 0.356 0.356) (layers "F.Cu" "F.Mask" "F.Paste") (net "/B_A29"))
  (pad "B30" smd circle (at -9.2075 -0.79) (size 0.356 0.356) (layers "F.Cu" "F.Mask" "F.Paste") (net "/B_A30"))
  (pad "C01" smd circle (at 9.2075 0.79) (size 0.356 0.356) (layers "F.Cu" "F.Mask" "F.Paste") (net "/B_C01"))
  (pad "C02" smd circle (at 8.572499 0.79) (size 0.356 0.356) (layers "F.Cu" "F.Mask" "F.Paste") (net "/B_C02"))
  (pad "C03" smd circle (at 7.9375 0.79) (size 0.356 0.356) (layers "F.Cu" "F.Mask" "F.Paste") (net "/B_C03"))
  (pad "C04" smd circle (at 7.3025 0.79) (size 0.356 0.356) (layers "F.Cu" "F.Mask" "F.Paste") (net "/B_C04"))
  (pad "C05" smd circle (at 6.667499 0.79) (size 0.356 0.356) (layers "F.Cu" "F.Mask" "F.Paste") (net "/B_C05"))
  (pad "C06" smd circle (at 6.0325 0.79) (size 0.356 0.356) (layers "F.Cu" "F.Mask" "F.Paste") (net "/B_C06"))
  (pad "C07" smd circle (at 5.3975 0.79) (size 0.356 0.356) (layers "F.Cu" "F.Mask" "F.Paste") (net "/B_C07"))
  (pad "C08" smd circle (at 4.762499 0.79) (size 0.356 0.356) (layers "F.Cu" "F.Mask" "F.Paste") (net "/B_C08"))
  (pad "C09" smd circle (at 4.1275 0.79) (size 0.356 0.356) (layers "F.Cu" "F.Mask" "F.Paste") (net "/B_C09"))
  (pad "C10" smd circle (at 3.4925 0.79) (size 0.356 0.356) (layers "F.Cu" "F.Mask" "F.Paste") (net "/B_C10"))
  (pad "C11" smd circle (at 2.8575 0.79) (size 0.356 0.356) (layers "F.Cu" "F.Mask" "F.Paste") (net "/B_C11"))
  (pad "C12" smd circle (at 2.2225 0.79) (size 0.356 0.356) (layers "F.Cu" "F.Mask" "F.Paste") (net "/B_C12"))
  (pad "C13" smd circle (at 1.5875 0.79) (size 0.356 0.356) (layers "F.Cu" "F.Mask" "F.Paste") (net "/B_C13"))
  (pad "C14" smd circle (at 0.9525 0.79) (size 0.356 0.356) (layers "F.Cu" "F.Mask" "F.Paste") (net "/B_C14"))
  (pad "C15" smd circle (at 0.3175 0.79) (size 0.356 0.356) (layers "F.Cu" "F.Mask" "F.Paste") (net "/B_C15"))
  (pad "C16" smd circle (at -0.3175 0.79) (size 0.356 0.356) (layers "F.Cu" "F.Mask" "F.Paste") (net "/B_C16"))
  (pad "C17" smd circle (at -0.9525 0.79) (size 0.356 0.356) (layers "F.Cu" "F.Mask" "F.Paste") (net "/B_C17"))
  (pad "C18" smd circle (at -1.5875 0.79) (size 0.356 0.356) (layers "F.Cu" "F.Mask" "F.Paste") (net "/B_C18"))
  (pad "C19" smd circle (at -2.2225 0.79) (size 0.356 0.356) (layers "F.Cu" "F.Mask" "F.Paste") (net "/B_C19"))
  (pad "C20" smd circle (at -2.8575 0.79) (size 0.356 0.356) (layers "F.Cu" "F.Mask" "F.Paste") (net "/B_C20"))
  (pad "C21" smd circle (at -3.4925 0.79) (size 0.356 0.356) (layers "F.Cu" "F.Mask" "F.Paste") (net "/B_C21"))
  (pad "C22" smd circle (at -4.1275 0.79) (size 0.356 0.356) (layers "F.Cu" "F.Mask" "F.Paste") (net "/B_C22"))
  (pad "C23" smd circle (at -4.7625 0.79) (size 0.356 0.356) (layers "F.Cu" "F.Mask" "F.Paste") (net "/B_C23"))
  (pad "C24" smd circle (at -5.3975 0.79) (size 0.356 0.356) (layers "F.Cu" "F.Mask" "F.Paste") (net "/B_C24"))
  (pad "C25" smd circle (at -6.0325 0.79) (size 0.356 0.356) (layers "F.Cu" "F.Mask" "F.Paste") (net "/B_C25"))
  (pad "C26" smd circle (at -6.6675 0.79) (size 0.356 0.356) (layers "F.Cu" "F.Mask" "F.Paste") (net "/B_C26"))
  (pad "C27" smd circle (at -7.3025 0.79) (size 0.356 0.356) (layers "F.Cu" "F.Mask" "F.Paste") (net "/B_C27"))
  (pad "C28" smd circle (at -7.9375 0.79) (size 0.356 0.356) (layers "F.Cu" "F.Mask" "F.Paste") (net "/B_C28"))
  (pad "C29" smd circle (at -8.5725 0.79) (size 0.356 0.356) (layers "F.Cu" "F.Mask" "F.Paste") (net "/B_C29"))
  (pad "C30" smd circle (at -9.2075 0.79) (size 0.356 0.356) (layers "F.Cu" "F.Mask" "F.Paste") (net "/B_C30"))
  (pad "D01" smd circle (at 9.2075 1.75) (size 0.356 0.356) (layers "F.Cu" "F.Mask" "F.Paste") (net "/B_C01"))
  (pad "D02" smd circle (at 8.572499 1.75) (size 0.356 0.356) (layers "F.Cu" "F.Mask" "F.Paste") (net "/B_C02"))
  (pad "D03" smd circle (at 7.9375 1.75) (size 0.356 0.356) (layers "F.Cu" "F.Mask" "F.Paste") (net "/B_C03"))
  (pad "D04" smd circle (at 7.3025 1.75) (size 0.356 0.356) (layers "F.Cu" "F.Mask" "F.Paste") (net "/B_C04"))
  (pad "D05" smd circle (at 6.667499 1.75) (size 0.356 0.356) (layers "F.Cu" "F.Mask" "F.Paste") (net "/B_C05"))
  (pad "D06" smd circle (at 6.0325 1.75) (size 0.356 0.356) (layers "F.Cu" "F.Mask" "F.Paste") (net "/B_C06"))
  (pad "D07" smd circle (at 5.3975 1.75) (size 0.356 0.356) (layers "F.Cu" "F.Mask" "F.Paste") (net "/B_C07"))
  (pad "D08" smd circle (at 4.762499 1.75) (size 0.356 0.356) (layers "F.Cu" "F.Mask" "F.Paste") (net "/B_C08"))
  (pad "D09" smd circle (at 4.1275 1.75) (size 0.356 0.356) (layers "F.Cu" "F.Mask" "F.Paste") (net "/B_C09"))
  (pad "D10" smd circle (at 3.4925 1.75) (size 0.356 0.356) (layers "F.Cu" "F.Mask" "F.Paste") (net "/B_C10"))
  (pad "D11" smd circle (at 2.8575 1.75) (size 0.356 0.356) (layers "F.Cu" "F.Mask" "F.Paste") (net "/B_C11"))
  (pad "D12" smd circle (at 2.2225 1.75) (size 0.356 0.356) (layers "F.Cu" "F.Mask" "F.Paste") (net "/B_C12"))
  (pad "D13" smd circle (at 1.5875 1.75) (size 0.356 0.356) (layers "F.Cu" "F.Mask" "F.Paste") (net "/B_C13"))
  (pad "D14" smd circle (at 0.9525 1.75) (size 0.356 0.356) (layers "F.Cu" "F.Mask" "F.Paste") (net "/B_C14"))
  (pad "D15" smd circle (at 0.3175 1.75) (size 0.356 0.356) (layers "F.Cu" "F.Mask" "F.Paste") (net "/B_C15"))
  (pad "D16" smd circle (at -0.3175 1.75) (size 0.356 0.356) (layers "F.Cu" "F.Mask" "F.Paste") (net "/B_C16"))
  (pad "D17" smd circle (at -0.9525 1.75) (size 0.356 0.356) (layers "F.Cu" "F.Mask" "F.Paste") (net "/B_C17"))
  (pad "D18" smd circle (at -1.5875 1.75) (size 0.356 0.356) (layers "F.Cu" "F.Mask" "F.Paste") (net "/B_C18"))
  (pad "D19" smd circle (at -2.2225 1.75) (size 0.356 0.356) (layers "F.Cu" "F.Mask" "F.Paste") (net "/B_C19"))
  (pad "D20" smd circle (at -2.8575 1.75) (size 0.356 0.356) (layers "F.Cu" "F.Mask" "F.Paste") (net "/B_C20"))
  (pad "D21" smd circle (at -3.4925 1.75) (size 0.356 0.356) (layers "F.Cu" "F.Mask" "F.Paste") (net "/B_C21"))
  (pad "D22" smd circle (at -4.1275 1.75) (size 0.356 0.356) (layers "F.Cu" "F.Mask" "F.Paste") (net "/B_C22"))
  (pad "D23" smd circle (at -4.7625 1.75) (size 0.356 0.356) (layers "F.Cu" "F.Mask" "F.Paste") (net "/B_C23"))
  (pad "D24" smd circle (at -5.3975 1.75) (size 0.356 0.356) (layers "F.Cu" "F.Mask" "F.Paste") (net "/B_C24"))
  (pad "D25" smd circle (at -6.0325 1.75) (size 0.356 0.356) (layers "F.Cu" "F.Mask" "F.Paste") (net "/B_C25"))
  (pad "D26" smd circle (at -6.6675 1.75) (size 0.356 0.356) (layers "F.Cu" "F.Mask" "F.Paste") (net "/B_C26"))
  (pad "D27" smd circle (at -7.3025 1.75) (size 0.356 0.356) (layers "F.Cu" "F.Mask" "F.Paste") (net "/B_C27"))
  (pad "D28" smd circle (at -7.9375 1.75) (size 0.356 0.356) (layers "F.Cu" "F.Mask" "F.Paste") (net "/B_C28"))
  (pad "D29" smd circle (at -8.5725 1.75) (size 0.356 0.356) (layers "F.Cu" "F.Mask" "F.Paste") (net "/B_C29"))
  (pad "D30" smd circle (at -9.2075 1.75) (size 0.356 0.356) (layers "F.Cu" "F.Mask" "F.Paste") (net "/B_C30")))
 (gr_rect (start 100 100) (end 150 140) (stroke (width 0.1) (type solid)) (fill no) (layer "Edge.Cuts"))
 (segment (start 134.2075 103.25) (end 134.2075 104.21) (width 0.2) (layer "F.Cu") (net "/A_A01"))
 (segment (start 133.572499 103.25) (end 133.572499 104.21) (width 0.2) (layer "F.Cu") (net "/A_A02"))
 (segment (start 132.9375 103.25) (end 132.9375 104.21) (width 0.2) (layer "F.Cu") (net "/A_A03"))
 (segment (start 132.3025 103.25) (end 132.3025 104.21) (width 0.2) (layer "F.Cu") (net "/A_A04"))
 (segment (start 131.667499 103.25) (end 131.667499 104.21) (width 0.2) (layer "F.Cu") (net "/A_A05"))
 (segment (start 131.0325 103.25) (end 131.0325 104.21) (width 0.2) (layer "F.Cu") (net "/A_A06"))
 (segment (start 130.3975 103.25) (end 130.3975 104.21) (width 0.2) (layer "F.Cu") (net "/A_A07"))
 (segment (start 129.762499 103.25) (end 129.762499 104.21) (width 0.2) (layer "F.Cu") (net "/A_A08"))
 (segment (start 129.1275 103.25) (end 129.1275 104.21) (width 0.2) (layer "F.Cu") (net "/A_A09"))
 (segment (start 128.4925 103.25) (end 128.4925 104.21) (width 0.2) (layer "F.Cu") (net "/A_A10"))
 (segment (start 127.8575 103.25) (end 127.8575 104.21) (width 0.2) (layer "F.Cu") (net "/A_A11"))
 (segment (start 127.2225 103.25) (end 127.2225 104.21) (width 0.2) (layer "F.Cu") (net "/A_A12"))
 (segment (start 126.5875 103.25) (end 126.5875 104.21) (width 0.2) (layer "F.Cu") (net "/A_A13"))
 (segment (start 125.9525 103.25) (end 125.9525 104.21) (width 0.2) (layer "F.Cu") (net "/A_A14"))
 (segment (start 125.3175 103.25) (end 125.3175 104.21) (width 0.2) (layer "F.Cu") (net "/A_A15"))
 (segment (start 124.6825 103.25) (end 124.6825 104.21) (width 0.2) (layer "F.Cu") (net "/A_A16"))
 (segment (start 124.0475 103.25) (end 124.0475 104.21) (width 0.2) (layer "F.Cu") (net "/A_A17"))
 (segment (start 123.4125 103.25) (end 123.4125 104.21) (width 0.2) (layer "F.Cu") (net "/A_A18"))
 (segment (start 122.7775 103.25) (end 122.7775 104.21) (width 0.2) (layer "F.Cu") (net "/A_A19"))
 (segment (start 122.1425 103.25) (end 122.1425 104.21) (width 0.2) (layer "F.Cu") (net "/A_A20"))
 (segment (start 121.5075 103.25) (end 121.5075 104.21) (width 0.2) (layer "F.Cu") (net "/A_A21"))
 (segment (start 120.8725 103.25) (end 120.8725 104.21) (width 0.2) (layer "F.Cu") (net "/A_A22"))
 (segment (start 120.2375 103.25) (end 120.2375 104.21) (width 0.2) (layer "F.Cu") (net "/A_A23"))
 (segment (start 119.6025 103.25) (end 119.6025 104.21) (width 0.2) (layer "F.Cu") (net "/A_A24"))
 (segment (start 118.9675 103.25) (end 118.9675 104.21) (width 0.2) (layer "F.Cu") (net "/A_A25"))
 (segment (start 118.3325 103.25) (end 118.3325 104.21) (width 0.2) (layer "F.Cu") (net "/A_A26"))
 (segment (start 117.6975 103.25) (end 117.6975 104.21) (width 0.2) (layer "F.Cu") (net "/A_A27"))
 (segment (start 117.0625 103.25) (end 117.0625 104.21) (width 0.2) (layer "F.Cu") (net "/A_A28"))
 (segment (start 116.4275 103.25) (end 116.4275 104.21) (width 0.2) (layer "F.Cu") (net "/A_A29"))
 (segment (start 115.7925 103.25) (end 115.7925 104.21) (width 0.2) (layer "F.Cu") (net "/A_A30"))
 (segment (start 134.2075 105.79) (end 134.2075 106.75) (width 0.2) (layer "F.Cu") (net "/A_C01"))
 (segment (start 133.572499 105.79) (end 133.572499 106.75) (width 0.2) (layer "F.Cu") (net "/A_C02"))
 (segment (start 132.9375 105.79) (end 132.9375 106.75) (width 0.2) (layer "F.Cu") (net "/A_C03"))
 (segment (start 132.3025 105.79) (end 132.3025 106.75) (width 0.2) (layer "F.Cu") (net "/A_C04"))
 (segment (start 131.667499 105.79) (end 131.667499 106.75) (width 0.2) (layer "F.Cu") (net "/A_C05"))
 (segment (start 131.0325 105.79) (end 131.0325 106.75) (width 0.2) (layer "F.Cu") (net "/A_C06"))
 (segment (start 130.3975 105.79) (end 130.3975 106.75) (width 0.2) (layer "F.Cu") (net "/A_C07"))
 (segment (start 129.762499 105.79) (end 129.762499 106.75) (width 0.2) (layer "F.Cu") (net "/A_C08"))
 (segment (start 129.1275 105.79) (end 129.1275 106.75) (width 0.2) (layer "F.Cu") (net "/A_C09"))
 (segment (start 128.4925 105.79) (end 128.4925 106.75) (width 0.2) (layer "F.Cu") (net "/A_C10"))
 (segment (start 127.8575 105.79) (end 127.8575 106.75) (width 0.2) (layer "F.Cu") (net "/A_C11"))
 (segment (start 127.2225 105.79) (end 127.2225 106.75) (width 0.2) (layer "F.Cu") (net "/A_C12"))
 (segment (start 126.5875 105.79) (end 126.5875 106.75) (width 0.2) (layer "F.Cu") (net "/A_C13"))
 (segment (start 125.9525 105.79) (end 125.9525 106.75) (width 0.2) (layer "F.Cu") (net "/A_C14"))
 (segment (start 125.3175 105.79) (end 125.3175 106.75) (width 0.2) (layer "F.Cu") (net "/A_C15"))
 (segment (start 124.6825 105.79) (end 124.6825 106.75) (width 0.2) (layer "F.Cu") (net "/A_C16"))
 (segment (start 124.0475 105.79) (end 124.0475 106.75) (width 0.2) (layer "F.Cu") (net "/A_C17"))
 (segment (start 123.4125 105.79) (end 123.4125 106.75) (width 0.2) (layer "F.Cu") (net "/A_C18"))
 (segment (start 122.7775 105.79) (end 122.7775 106.75) (width 0.2) (layer "F.Cu") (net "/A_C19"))
 (segment (start 122.1425 105.79) (end 122.1425 106.75) (width 0.2) (layer "F.Cu") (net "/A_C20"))
 (segment (start 121.5075 105.79) (end 121.5075 106.75) (width 0.2) (layer "F.Cu") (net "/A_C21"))
 (segment (start 120.8725 105.79) (end 120.8725 106.75) (width 0.2) (layer "F.Cu") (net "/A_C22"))
 (segment (start 120.2375 105.79) (end 120.2375 106.75) (width 0.2) (layer "F.Cu") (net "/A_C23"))
 (segment (start 119.6025 105.79) (end 119.6025 106.75) (width 0.2) (layer "F.Cu") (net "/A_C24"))
 (segment (start 118.9675 105.79) (end 118.9675 106.75) (width 0.2) (layer "F.Cu") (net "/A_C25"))
 (segment (start 118.3325 105.79) (end 118.3325 106.75) (width 0.2) (layer "F.Cu") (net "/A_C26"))
 (segment (start 117.6975 105.79) (end 117.6975 106.75) (width 0.2) (layer "F.Cu") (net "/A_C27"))
 (segment (start 117.0625 105.79) (end 117.0625 106.75) (width 0.2) (layer "F.Cu") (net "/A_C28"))
 (segment (start 116.4275 105.79) (end 116.4275 106.75) (width 0.2) (layer "F.Cu") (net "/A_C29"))
 (segment (start 115.7925 105.79) (end 115.7925 106.75) (width 0.2) (layer "F.Cu") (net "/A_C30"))
 (segment (start 134.2075 133.25) (end 134.2075 134.21) (width 0.2) (layer "F.Cu") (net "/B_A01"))
 (segment (start 133.572499 133.25) (end 133.572499 134.21) (width 0.2) (layer "F.Cu") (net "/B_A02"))
 (segment (start 132.9375 133.25) (end 132.9375 134.21) (width 0.2) (layer "F.Cu") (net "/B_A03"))
 (segment (start 132.3025 133.25) (end 132.3025 134.21) (width 0.2) (layer "F.Cu") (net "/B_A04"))
 (segment (start 131.667499 133.25) (end 131.667499 134.21) (width 0.2) (layer "F.Cu") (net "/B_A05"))
 (segment (start 131.0325 133.25) (end 131.0325 134.21) (width 0.2) (layer "F.Cu") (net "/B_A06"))
 (segment (start 130.3975 133.25) (end 130.3975 134.21) (width 0.2) (layer "F.Cu") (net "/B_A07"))
 (segment (start 129.762499 133.25) (end 129.762499 134.21) (width 0.2) (layer "F.Cu") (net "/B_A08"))
 (segment (start 129.1275 133.25) (end 129.1275 134.21) (width 0.2) (layer "F.Cu") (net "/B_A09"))
 (segment (start 128.4925 133.25) (end 128.4925 134.21) (width 0.2) (layer "F.Cu") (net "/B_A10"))
 (segment (start 127.8575 133.25) (end 127.8575 134.21) (width 0.2) (layer "F.Cu") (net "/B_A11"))
 (segment (start 127.2225 133.25) (end 127.2225 134.21) (width 0.2) (layer "F.Cu") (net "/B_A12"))
 (segment (start 126.5875 133.25) (end 126.5875 134.21) (width 0.2) (layer "F.Cu") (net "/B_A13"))
 (segment (start 125.9525 133.25) (end 125.9525 134.21) (width 0.2) (layer "F.Cu") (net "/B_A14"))
 (segment (start 125.3175 133.25) (end 125.3175 134.21) (width 0.2) (layer "F.Cu") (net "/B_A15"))
 (segment (start 124.6825 133.25) (end 124.6825 134.21) (width 0.2) (layer "F.Cu") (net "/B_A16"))
 (segment (start 124.0475 133.25) (end 124.0475 134.21) (width 0.2) (layer "F.Cu") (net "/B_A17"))
 (segment (start 123.4125 133.25) (end 123.4125 134.21) (width 0.2) (layer "F.Cu") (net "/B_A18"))
 (segment (start 122.7775 133.25) (end 122.7775 134.21) (width 0.2) (layer "F.Cu") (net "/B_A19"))
 (segment (start 122.1425 133.25) (end 122.1425 134.21) (width 0.2) (layer "F.Cu") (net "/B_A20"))
 (segment (start 121.5075 133.25) (end 121.5075 134.21) (width 0.2) (layer "F.Cu") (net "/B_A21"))
 (segment (start 120.8725 133.25) (end 120.8725 134.21) (width 0.2) (layer "F.Cu") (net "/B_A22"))
 (segment (start 120.2375 133.25) (end 120.2375 134.21) (width 0.2) (layer "F.Cu") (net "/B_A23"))
 (segment (start 119.6025 133.25) (end 119.6025 134.21) (width 0.2) (layer "F.Cu") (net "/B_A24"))
 (segment (start 118.9675 133.25) (end 118.9675 134.21) (width 0.2) (layer "F.Cu") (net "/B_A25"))
 (segment (start 118.3325 133.25) (end 118.3325 134.21) (width 0.2) (layer "F.Cu") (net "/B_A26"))
 (segment (start 117.6975 133.25) (end 117.6975 134.21) (width 0.2) (layer "F.Cu") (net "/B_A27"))
 (segment (start 117.0625 133.25) (end 117.0625 134.21) (width 0.2) (layer "F.Cu") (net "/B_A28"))
 (segment (start 116.4275 133.25) (end 116.4275 134.21) (width 0.2) (layer "F.Cu") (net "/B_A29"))
 (segment (start 115.7925 133.25) (end 115.7925 134.21) (width 0.2) (layer "F.Cu") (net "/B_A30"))
 (segment (start 134.2075 135.79) (end 134.2075 136.75) (width 0.2) (layer "F.Cu") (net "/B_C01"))
 (segment (start 133.572499 135.79) (end 133.572499 136.75) (width 0.2) (layer "F.Cu") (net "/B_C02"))
 (segment (start 132.9375 135.79) (end 132.9375 136.75) (width 0.2) (layer "F.Cu") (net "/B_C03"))
 (segment (start 132.3025 135.79) (end 132.3025 136.75) (width 0.2) (layer "F.Cu") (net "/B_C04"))
 (segment (start 131.667499 135.79) (end 131.667499 136.75) (width 0.2) (layer "F.Cu") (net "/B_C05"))
 (segment (start 131.0325 135.79) (end 131.0325 136.75) (width 0.2) (layer "F.Cu") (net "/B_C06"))
 (segment (start 130.3975 135.79) (end 130.3975 136.75) (width 0.2) (layer "F.Cu") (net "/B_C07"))
 (segment (start 129.762499 135.79) (end 129.762499 136.75) (width 0.2) (layer "F.Cu") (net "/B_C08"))
 (segment (start 129.1275 135.79) (end 129.1275 136.75) (width 0.2) (layer "F.Cu") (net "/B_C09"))
 (segment (start 128.4925 135.79) (end 128.4925 136.75) (width 0.2) (layer "F.Cu") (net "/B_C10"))
 (segment (start 127.8575 135.79) (end 127.8575 136.75) (width 0.2) (layer "F.Cu") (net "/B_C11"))
 (segment (start 127.2225 135.79) (end 127.2225 136.75) (width 0.2) (layer "F.Cu") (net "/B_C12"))
 (segment (start 126.5875 135.79) (end 126.5875 136.75) (width 0.2) (layer "F.Cu") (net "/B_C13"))
 (segment (start 125.9525 135.79) (end 125.9525 136.75) (width 0.2) (layer "F.Cu") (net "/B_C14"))
 (segment (start 125.3175 135.79) (end 125.3175 136.75) (width 0.2) (layer "F.Cu") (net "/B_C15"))
 (segment (start 124.6825 135.79) (end 124.6825 136.75) (width 0.2) (layer "F.Cu") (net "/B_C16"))
 (segment (start 124.0475 135.79) (end 124.0475 136.75) (width 0.2) (layer "F.Cu") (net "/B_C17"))
 (segment (start 123.4125 135.79) (end 123.4125 136.75) (width 0.2) (layer "F.Cu") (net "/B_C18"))
 (segment (start 122.7775 135.79) (end 122.7775 136.75) (width 0.2) (layer "F.Cu") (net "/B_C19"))
 (segment (start 122.1425 135.79) (end 122.1425 136.75) (width 0.2) (layer "F.Cu") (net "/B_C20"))
 (segment (start 121.5075 135.79) (end 121.5075 136.75) (width 0.2) (layer "F.Cu") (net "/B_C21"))
 (segment (start 120.8725 135.79) (end 120.8725 136.75) (width 0.2) (layer "F.Cu") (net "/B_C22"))
 (segment (start 120.2375 135.79) (end 120.2375 136.75) (width 0.2) (layer "F.Cu") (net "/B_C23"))
 (segment (start 119.6025 135.79) (end 119.6025 136.75) (width 0.2) (layer "F.Cu") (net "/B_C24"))
 (segment (start 118.9675 135.79) (end 118.9675 136.75) (width 0.2) (layer "F.Cu") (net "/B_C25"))
 (segment (start 118.3325 135.79) (end 118.3325 136.75) (width 0.2) (layer "F.Cu") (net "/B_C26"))
 (segment (start 117.6975 135.79) (end 117.6975 136.75) (width 0.2) (layer "F.Cu") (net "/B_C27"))
 (segment (start 117.0625 135.79) (end 117.0625 136.75) (width 0.2) (layer "F.Cu") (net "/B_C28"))
 (segment (start 116.4275 135.79) (end 116.4275 136.75) (width 0.2) (layer "F.Cu") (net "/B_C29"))
 (segment (start 115.7925 135.79) (end 115.7925 136.75) (width 0.2) (layer "F.Cu") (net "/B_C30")))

